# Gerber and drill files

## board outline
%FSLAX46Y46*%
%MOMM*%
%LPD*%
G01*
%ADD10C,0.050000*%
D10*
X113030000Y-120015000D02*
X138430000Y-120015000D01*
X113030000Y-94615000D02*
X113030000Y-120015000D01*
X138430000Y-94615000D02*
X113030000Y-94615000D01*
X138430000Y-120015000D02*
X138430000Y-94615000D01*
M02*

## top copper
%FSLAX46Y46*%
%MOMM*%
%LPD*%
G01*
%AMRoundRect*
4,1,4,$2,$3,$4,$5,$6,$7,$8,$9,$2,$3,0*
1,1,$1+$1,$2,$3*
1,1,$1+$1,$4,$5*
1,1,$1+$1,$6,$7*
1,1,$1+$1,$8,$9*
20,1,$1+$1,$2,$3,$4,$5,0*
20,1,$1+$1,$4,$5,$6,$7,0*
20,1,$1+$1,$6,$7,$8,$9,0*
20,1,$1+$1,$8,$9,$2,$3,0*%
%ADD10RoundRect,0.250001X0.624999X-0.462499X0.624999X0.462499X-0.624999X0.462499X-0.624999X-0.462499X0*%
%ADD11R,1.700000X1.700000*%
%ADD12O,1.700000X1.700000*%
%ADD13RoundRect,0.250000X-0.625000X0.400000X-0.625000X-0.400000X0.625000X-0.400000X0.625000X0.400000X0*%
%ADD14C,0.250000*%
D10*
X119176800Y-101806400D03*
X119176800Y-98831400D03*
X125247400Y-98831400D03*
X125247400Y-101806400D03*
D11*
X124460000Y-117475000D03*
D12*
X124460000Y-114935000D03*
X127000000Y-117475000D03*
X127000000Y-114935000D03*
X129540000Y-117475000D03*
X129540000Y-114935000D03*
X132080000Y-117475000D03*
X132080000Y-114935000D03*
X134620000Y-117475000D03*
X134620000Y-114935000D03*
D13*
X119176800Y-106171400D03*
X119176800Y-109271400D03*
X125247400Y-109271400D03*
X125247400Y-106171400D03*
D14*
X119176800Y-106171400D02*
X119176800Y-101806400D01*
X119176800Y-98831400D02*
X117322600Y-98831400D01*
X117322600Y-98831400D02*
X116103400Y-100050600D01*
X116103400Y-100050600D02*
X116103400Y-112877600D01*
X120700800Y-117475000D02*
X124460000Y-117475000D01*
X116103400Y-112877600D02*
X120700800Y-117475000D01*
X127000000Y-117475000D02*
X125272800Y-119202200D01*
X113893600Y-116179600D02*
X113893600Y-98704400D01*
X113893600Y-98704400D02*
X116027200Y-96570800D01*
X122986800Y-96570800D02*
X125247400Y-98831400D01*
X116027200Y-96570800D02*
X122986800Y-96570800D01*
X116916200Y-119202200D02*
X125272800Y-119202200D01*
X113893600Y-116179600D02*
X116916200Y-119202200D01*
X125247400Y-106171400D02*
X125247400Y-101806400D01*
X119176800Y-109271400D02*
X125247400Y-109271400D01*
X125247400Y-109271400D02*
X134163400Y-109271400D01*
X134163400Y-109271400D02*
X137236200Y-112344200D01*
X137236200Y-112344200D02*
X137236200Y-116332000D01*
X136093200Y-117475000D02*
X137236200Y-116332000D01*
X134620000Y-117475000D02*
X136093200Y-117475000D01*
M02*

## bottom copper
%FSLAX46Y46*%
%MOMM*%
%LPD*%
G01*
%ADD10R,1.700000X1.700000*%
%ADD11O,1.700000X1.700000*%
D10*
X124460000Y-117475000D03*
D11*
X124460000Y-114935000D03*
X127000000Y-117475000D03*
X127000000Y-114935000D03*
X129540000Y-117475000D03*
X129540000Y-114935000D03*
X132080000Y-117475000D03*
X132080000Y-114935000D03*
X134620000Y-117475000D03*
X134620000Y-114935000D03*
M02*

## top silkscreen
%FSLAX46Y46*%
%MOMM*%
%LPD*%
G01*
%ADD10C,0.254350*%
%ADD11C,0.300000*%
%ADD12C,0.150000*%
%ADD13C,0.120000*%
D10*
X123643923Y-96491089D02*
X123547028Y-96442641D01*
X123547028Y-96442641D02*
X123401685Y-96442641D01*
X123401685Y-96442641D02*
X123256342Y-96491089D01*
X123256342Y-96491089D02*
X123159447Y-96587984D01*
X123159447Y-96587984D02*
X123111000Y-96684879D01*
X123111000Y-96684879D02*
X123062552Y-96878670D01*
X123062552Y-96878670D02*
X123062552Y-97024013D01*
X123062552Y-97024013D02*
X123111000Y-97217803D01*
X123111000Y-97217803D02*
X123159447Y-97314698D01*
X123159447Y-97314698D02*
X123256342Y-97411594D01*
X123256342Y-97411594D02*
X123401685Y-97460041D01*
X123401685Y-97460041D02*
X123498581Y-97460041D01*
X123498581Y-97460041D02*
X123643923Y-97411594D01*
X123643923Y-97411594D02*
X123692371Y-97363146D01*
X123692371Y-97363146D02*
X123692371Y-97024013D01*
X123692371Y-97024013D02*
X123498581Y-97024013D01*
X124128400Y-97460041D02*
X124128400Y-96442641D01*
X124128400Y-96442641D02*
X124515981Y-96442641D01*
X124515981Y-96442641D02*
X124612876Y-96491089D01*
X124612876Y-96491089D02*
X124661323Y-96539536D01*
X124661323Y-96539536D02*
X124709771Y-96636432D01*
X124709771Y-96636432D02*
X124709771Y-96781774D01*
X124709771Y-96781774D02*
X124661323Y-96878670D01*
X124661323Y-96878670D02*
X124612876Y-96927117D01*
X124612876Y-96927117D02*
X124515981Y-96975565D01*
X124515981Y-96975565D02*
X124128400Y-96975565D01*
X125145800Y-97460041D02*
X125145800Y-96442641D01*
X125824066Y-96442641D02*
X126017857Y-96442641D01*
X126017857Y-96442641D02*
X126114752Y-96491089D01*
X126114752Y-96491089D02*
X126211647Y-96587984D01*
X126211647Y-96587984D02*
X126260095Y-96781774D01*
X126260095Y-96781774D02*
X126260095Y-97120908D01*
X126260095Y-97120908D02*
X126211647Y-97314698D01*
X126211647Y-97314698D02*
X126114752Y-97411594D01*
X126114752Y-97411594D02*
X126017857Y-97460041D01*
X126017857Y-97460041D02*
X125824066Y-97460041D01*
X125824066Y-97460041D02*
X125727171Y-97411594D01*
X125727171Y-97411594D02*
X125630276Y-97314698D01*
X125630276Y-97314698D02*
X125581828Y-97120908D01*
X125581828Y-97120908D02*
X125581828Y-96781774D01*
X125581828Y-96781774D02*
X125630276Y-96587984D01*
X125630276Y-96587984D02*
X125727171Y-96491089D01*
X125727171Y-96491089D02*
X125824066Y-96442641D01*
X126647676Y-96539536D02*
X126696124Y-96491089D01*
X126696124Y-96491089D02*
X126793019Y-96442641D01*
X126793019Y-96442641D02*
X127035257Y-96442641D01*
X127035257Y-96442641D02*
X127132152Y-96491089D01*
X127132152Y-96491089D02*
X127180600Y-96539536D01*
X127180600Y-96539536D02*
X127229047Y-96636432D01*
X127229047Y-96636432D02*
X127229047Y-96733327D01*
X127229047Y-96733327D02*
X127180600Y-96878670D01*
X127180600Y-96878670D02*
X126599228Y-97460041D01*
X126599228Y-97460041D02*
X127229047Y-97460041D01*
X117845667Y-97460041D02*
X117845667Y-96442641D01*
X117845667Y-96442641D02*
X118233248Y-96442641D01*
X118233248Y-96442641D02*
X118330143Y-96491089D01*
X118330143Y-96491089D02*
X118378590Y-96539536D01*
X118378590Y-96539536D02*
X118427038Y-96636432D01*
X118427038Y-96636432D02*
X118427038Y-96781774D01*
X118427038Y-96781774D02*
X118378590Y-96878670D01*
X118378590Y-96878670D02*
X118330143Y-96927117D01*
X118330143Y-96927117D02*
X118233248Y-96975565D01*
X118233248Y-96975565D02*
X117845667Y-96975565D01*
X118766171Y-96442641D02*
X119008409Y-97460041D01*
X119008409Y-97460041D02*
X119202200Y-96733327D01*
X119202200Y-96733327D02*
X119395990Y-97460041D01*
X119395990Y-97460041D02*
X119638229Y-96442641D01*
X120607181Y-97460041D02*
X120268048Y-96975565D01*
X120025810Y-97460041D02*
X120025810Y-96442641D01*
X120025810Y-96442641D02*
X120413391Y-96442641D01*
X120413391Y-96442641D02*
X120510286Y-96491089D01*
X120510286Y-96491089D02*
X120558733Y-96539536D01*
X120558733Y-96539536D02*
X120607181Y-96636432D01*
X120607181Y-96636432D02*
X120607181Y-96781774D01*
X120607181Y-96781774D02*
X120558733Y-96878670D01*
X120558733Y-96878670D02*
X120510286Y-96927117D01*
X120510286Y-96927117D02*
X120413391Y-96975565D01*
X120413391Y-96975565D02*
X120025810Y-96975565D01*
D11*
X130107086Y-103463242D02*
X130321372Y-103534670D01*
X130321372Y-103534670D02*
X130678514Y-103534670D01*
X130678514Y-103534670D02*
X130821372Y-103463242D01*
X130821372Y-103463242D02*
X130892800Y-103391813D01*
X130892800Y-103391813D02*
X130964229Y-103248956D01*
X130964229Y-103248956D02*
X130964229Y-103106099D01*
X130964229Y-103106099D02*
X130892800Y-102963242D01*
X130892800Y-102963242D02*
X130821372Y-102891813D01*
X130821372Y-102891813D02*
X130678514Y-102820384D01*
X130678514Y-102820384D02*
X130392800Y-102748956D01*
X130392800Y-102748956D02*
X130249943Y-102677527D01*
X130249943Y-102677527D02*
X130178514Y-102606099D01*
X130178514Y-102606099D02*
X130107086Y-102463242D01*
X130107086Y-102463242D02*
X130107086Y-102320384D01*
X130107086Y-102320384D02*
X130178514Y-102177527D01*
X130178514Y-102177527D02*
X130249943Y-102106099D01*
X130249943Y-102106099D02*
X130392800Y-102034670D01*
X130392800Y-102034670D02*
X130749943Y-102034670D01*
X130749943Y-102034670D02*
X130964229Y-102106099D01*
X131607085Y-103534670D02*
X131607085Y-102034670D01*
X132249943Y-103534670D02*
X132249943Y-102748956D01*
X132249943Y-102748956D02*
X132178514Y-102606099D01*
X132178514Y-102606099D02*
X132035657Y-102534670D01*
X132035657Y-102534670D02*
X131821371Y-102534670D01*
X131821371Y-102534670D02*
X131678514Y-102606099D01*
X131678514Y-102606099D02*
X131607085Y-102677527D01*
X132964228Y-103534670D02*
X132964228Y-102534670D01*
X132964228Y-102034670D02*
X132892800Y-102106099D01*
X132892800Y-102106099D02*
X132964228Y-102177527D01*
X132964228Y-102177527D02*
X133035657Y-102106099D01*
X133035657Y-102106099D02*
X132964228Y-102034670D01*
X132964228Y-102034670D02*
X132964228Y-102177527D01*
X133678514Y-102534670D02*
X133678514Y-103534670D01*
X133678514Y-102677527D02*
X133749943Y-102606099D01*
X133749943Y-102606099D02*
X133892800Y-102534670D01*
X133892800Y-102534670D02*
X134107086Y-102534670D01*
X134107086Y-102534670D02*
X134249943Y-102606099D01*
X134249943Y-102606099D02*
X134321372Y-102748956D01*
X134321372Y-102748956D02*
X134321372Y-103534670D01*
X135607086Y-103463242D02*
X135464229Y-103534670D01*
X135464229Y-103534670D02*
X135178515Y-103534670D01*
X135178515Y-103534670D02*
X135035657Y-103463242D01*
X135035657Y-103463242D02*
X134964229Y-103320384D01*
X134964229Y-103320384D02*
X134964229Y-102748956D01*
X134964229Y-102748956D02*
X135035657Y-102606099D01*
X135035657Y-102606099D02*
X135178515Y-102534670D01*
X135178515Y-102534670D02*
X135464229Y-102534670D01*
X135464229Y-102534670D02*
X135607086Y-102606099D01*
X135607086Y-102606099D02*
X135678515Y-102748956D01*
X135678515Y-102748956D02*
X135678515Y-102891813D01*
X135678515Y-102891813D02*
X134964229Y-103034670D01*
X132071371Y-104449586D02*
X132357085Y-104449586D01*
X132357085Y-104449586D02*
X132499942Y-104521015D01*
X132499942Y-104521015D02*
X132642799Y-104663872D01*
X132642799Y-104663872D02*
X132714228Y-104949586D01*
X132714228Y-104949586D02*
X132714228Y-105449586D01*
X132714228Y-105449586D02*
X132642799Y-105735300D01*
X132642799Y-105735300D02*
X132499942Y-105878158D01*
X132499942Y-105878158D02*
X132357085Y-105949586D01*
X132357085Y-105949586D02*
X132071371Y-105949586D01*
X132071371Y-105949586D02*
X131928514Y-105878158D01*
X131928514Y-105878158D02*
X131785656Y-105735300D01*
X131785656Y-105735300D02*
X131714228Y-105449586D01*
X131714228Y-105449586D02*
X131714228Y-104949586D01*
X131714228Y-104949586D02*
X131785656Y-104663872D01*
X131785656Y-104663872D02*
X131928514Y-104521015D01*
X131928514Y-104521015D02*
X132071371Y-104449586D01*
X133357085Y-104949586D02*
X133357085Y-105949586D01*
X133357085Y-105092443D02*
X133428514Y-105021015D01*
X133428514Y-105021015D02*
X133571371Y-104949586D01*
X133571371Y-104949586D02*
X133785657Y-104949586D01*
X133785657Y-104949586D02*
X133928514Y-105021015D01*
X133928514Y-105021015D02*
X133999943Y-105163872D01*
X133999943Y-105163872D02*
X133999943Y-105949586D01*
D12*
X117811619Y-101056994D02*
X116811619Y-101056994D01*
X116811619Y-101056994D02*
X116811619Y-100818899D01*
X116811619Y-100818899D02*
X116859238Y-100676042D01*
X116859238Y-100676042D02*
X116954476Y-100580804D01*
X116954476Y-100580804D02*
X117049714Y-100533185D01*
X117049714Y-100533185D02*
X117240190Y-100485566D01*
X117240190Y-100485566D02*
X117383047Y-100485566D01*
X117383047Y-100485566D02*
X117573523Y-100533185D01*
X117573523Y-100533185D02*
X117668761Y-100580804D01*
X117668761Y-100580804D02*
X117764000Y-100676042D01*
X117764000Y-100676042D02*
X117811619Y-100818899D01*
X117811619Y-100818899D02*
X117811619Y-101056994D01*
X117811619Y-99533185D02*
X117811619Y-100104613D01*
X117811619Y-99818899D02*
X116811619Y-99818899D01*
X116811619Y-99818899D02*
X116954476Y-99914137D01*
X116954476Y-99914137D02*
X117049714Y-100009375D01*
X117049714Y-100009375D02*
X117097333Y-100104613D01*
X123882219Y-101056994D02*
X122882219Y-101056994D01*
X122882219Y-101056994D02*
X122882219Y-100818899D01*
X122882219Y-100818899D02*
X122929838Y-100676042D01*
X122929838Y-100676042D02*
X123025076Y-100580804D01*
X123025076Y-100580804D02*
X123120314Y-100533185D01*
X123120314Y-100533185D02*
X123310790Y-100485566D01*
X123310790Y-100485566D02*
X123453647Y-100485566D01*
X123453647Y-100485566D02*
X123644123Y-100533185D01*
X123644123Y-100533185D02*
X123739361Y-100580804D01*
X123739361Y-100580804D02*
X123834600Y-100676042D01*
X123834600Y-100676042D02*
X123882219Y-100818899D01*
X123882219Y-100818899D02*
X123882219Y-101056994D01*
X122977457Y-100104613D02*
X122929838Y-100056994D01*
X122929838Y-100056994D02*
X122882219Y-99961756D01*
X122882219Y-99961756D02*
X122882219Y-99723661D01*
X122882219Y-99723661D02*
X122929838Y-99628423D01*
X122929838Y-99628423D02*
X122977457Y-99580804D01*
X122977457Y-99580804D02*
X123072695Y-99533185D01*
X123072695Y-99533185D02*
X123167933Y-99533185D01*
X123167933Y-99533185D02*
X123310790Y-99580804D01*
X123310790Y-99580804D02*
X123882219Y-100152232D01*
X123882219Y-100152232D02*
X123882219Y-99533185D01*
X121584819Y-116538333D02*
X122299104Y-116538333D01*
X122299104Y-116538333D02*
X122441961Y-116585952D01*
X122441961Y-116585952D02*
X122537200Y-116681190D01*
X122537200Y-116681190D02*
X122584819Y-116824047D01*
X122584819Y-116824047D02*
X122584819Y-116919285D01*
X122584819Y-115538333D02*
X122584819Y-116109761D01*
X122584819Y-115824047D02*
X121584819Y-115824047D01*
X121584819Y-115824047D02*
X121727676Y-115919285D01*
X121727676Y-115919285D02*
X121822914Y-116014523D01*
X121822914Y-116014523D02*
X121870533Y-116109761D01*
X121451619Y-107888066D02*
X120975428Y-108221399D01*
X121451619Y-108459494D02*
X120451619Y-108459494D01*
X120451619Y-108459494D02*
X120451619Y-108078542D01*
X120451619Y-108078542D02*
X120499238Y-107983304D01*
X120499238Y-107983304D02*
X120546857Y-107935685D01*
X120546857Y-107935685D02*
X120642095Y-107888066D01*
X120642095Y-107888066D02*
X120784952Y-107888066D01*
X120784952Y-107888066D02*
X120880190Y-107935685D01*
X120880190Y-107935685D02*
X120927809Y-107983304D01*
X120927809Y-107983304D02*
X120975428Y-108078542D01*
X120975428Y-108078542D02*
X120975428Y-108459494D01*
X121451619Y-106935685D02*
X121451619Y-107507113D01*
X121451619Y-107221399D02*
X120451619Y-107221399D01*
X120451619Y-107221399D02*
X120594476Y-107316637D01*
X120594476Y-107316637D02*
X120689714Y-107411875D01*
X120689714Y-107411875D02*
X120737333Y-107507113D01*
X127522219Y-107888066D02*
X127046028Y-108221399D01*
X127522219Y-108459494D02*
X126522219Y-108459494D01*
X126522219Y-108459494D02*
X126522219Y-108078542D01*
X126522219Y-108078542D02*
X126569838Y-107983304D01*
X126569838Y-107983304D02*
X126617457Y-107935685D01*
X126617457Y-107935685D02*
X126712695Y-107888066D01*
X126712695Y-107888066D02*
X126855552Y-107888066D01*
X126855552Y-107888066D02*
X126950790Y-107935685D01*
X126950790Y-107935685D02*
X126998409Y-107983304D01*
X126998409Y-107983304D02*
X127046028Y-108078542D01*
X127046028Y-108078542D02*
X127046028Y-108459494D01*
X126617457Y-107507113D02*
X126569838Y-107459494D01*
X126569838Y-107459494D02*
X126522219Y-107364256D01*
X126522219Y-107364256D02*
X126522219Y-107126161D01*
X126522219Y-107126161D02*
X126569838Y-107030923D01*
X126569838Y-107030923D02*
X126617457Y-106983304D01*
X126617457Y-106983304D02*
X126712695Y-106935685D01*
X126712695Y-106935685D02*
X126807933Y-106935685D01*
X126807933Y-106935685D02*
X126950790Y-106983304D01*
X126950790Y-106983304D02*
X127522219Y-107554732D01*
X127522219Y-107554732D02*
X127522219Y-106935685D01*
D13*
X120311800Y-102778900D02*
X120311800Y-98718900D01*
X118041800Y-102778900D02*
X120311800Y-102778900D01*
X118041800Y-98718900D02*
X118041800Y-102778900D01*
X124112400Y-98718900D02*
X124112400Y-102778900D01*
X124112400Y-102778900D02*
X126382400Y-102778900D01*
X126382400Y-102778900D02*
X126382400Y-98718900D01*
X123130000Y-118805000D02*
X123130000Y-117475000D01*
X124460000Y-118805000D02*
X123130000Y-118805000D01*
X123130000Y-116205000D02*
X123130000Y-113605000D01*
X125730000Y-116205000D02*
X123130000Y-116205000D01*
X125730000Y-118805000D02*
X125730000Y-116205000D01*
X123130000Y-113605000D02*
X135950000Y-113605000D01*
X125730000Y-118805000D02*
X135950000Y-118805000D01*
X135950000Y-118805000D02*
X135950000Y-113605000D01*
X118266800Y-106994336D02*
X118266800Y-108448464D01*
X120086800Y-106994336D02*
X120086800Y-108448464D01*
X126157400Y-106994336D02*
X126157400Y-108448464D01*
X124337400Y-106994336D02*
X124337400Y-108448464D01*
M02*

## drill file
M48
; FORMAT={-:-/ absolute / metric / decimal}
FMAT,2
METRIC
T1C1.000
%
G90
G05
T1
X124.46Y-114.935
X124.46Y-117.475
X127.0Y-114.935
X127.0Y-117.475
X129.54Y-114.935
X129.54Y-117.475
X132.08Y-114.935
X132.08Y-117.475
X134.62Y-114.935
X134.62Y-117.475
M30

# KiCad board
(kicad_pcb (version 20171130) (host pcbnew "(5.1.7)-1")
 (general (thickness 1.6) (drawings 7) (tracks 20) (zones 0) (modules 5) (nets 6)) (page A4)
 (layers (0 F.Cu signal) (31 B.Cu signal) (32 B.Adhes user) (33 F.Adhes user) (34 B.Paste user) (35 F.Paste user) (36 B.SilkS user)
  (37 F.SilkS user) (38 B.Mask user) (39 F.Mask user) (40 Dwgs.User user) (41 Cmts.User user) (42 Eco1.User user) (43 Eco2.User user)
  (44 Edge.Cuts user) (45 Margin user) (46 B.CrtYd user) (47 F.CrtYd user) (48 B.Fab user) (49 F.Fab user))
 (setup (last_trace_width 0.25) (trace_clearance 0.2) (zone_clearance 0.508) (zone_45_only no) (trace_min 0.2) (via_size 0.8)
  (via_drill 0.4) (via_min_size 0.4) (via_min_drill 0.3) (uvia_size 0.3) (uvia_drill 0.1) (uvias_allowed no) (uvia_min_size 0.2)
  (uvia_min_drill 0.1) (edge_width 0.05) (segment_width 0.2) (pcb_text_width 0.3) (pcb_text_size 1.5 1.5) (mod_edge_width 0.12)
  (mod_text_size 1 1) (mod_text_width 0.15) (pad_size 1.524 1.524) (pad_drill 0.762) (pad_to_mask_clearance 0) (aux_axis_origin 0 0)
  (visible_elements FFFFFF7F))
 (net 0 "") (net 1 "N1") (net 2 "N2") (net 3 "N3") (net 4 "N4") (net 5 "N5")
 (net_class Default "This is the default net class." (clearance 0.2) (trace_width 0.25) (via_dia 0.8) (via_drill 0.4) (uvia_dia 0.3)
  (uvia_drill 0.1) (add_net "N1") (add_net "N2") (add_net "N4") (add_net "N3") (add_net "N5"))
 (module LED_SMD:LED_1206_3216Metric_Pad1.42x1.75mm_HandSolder (layer F.Cu) (at 119.1768 100.3189 90)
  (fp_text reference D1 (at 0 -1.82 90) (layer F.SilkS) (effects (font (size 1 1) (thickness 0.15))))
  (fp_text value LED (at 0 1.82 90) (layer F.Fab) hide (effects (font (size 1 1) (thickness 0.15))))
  (fp_line (start -2.46 1.135) (end 1.6 1.135) (layer F.SilkS) (width 0.12))
  (fp_line (start -2.46 -1.135) (end -2.46 1.135) (layer F.SilkS) (width 0.12))
  (fp_line (start 1.6 -1.135) (end -2.46 -1.135) (layer F.SilkS) (width 0.12))
  (pad 1 smd roundrect (at -1.4875 0 90) (size 1.425 1.75) (layers F.Cu F.Paste F.Mask) (roundrect_rratio 0.175439) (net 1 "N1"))
  (pad 2 smd roundrect (at 1.4875 0 90) (size 1.425 1.75) (layers F.Cu F.Paste F.Mask) (roundrect_rratio 0.175439) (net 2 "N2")))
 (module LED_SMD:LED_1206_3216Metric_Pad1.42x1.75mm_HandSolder (layer F.Cu) (at 125.2474 100.3189 90)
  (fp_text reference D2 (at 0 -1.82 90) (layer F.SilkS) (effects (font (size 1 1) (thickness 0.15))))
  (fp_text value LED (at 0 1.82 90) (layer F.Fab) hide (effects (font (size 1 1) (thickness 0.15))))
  (fp_line (start 1.6 -1.135) (end -2.46 -1.135) (layer F.SilkS) (width 0.12))
  (fp_line (start -2.46 -1.135) (end -2.46 1.135) (layer F.SilkS) (width 0.12))
  (fp_line (start -2.46 1.135) (end 1.6 1.135) (layer F.SilkS) (width 0.12))
  (pad 2 smd roundrect (at 1.4875 0 90) (size 1.425 1.75) (layers F.Cu F.Paste F.Mask) (roundrect_rratio 0.175439) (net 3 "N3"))
  (pad 1 smd roundrect (at -1.4875 0 90) (size 1.425 1.75) (layers F.Cu F.Paste F.Mask) (roundrect_rratio 0.175439) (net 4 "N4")))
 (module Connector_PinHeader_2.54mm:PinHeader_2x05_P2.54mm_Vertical (layer F.Cu) (at 124.46 117.475 90)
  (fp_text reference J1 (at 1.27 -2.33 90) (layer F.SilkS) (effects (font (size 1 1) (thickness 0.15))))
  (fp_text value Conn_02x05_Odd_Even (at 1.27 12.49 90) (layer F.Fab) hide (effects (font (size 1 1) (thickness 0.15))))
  (fp_line (start -1.33 -1.33) (end 0 -1.33) (layer F.SilkS) (width 0.12))
  (fp_line (start -1.33 0) (end -1.33 -1.33) (layer F.SilkS) (width 0.12))
  (fp_line (start 1.27 -1.33) (end 3.87 -1.33) (layer F.SilkS) (width 0.12))
  (fp_line (start 1.27 1.27) (end 1.27 -1.33) (layer F.SilkS) (width 0.12))
  (fp_line (start -1.33 1.27) (end 1.27 1.27) (layer F.SilkS) (width 0.12))
  (fp_line (start 3.87 -1.33) (end 3.87 11.49) (layer F.SilkS) (width 0.12))
  (fp_line (start -1.33 1.27) (end -1.33 11.49) (layer F.SilkS) (width 0.12))
  (fp_line (start -1.33 11.49) (end 3.87 11.49) (layer F.SilkS) (width 0.12))
  (pad 1 thru_hole rect (at 0 0 90) (size 1.7 1.7) (drill 1) (layers *.Cu *.Mask) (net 2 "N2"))
  (pad 2 thru_hole oval (at 2.54 0 90) (size 1.7 1.7) (drill 1) (layers *.Cu *.Mask))
  (pad 3 thru_hole oval (at 0 2.54 90) (size 1.7 1.7) (drill 1) (layers *.Cu *.Mask) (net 3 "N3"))
  (pad 4 thru_hole oval (at 2.54 2.54 90) (size 1.7 1.7) (drill 1) (layers *.Cu *.Mask))
  (pad 5 thru_hole oval (at 0 5.08 90) (size 1.7 1.7) (drill 1) (layers *.Cu *.Mask))
  (pad 6 thru_hole oval (at 2.54 5.08 90) (size 1.7 1.7) (drill 1) (layers *.Cu *.Mask))
  (pad 7 thru_hole oval (at 0 7.62 90) (size 1.7 1.7) (drill 1) (layers *.Cu *.Mask))
  (pad 8 thru_hole oval (at 2.54 7.62 90) (size 1.7 1.7) (drill 1) (layers *.Cu *.Mask))
  (pad 9 thru_hole oval (at 0 10.16 90) (size 1.7 1.7) (drill 1) (layers *.Cu *.Mask) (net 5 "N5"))
  (pad 10 thru_hole oval (at 2.54 10.16 90) (size 1.7 1.7) (drill 1) (layers *.Cu *.Mask)))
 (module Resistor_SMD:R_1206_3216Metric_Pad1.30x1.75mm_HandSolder (layer F.Cu) (at 119.1768 107.7214 270)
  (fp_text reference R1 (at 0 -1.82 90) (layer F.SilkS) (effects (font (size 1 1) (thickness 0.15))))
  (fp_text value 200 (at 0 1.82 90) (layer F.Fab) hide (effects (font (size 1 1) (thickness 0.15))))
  (fp_line (start -0.727064 0.91) (end 0.727064 0.91) (layer F.SilkS) (width 0.12))
  (fp_line (start -0.727064 -0.91) (end 0.727064 -0.91) (layer F.SilkS) (width 0.12))
  (pad 1 smd roundrect (at -1.55 0 270) (size 1.3 1.75) (layers F.Cu F.Paste F.Mask) (roundrect_rratio 0.192308) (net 1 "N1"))
  (pad 2 smd roundrect (at 1.55 0 270) (size 1.3 1.75) (layers F.Cu F.Paste F.Mask) (roundrect_rratio 0.192308) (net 5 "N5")))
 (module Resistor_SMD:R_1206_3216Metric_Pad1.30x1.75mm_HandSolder (layer F.Cu) (at 125.2474 107.7214 270)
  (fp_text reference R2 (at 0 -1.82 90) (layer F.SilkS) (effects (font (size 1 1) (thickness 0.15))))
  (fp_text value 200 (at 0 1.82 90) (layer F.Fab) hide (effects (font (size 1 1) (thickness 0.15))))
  (fp_line (start -0.727064 -0.91) (end 0.727064 -0.91) (layer F.SilkS) (width 0.12))
  (fp_line (start -0.727064 0.91) (end 0.727064 0.91) (layer F.SilkS) (width 0.12))
  (pad 2 smd roundrect (at 1.55 0 270) (size 1.3 1.75) (layers F.Cu F.Paste F.Mask) (roundrect_rratio 0.192308) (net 5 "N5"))
  (pad 1 smd roundrect (at -1.55 0 270) (size 1.3 1.75) (layers F.Cu F.Paste F.Mask) (roundrect_rratio 0.192308) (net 4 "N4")))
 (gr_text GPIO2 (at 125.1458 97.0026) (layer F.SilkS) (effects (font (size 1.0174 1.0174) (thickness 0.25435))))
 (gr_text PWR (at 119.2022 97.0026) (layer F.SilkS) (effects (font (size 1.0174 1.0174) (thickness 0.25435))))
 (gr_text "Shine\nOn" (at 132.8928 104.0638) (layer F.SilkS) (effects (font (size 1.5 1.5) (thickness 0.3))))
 (gr_line (start 113.03 120.015) (end 138.43 120.015) (layer Edge.Cuts) (width 0.05))
 (gr_line (start 113.03 94.615) (end 113.03 120.015) (layer Edge.Cuts) (width 0.05))
 (gr_line (start 138.43 94.615) (end 113.03 94.615) (layer Edge.Cuts) (width 0.05))
 (gr_line (start 138.43 120.015) (end 138.43 94.615) (layer Edge.Cuts) (width 0.05))
 (segment (start 119.1768 106.1714) (end 119.1768 101.8064) (width 0.25) (layer F.Cu) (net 1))
 (segment (start 119.1768 98.8314) (end 117.3226 98.8314) (width 0.25) (layer F.Cu) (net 2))
 (segment (start 117.3226 98.8314) (end 116.1034 100.0506) (width 0.25) (layer F.Cu) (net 2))
 (segment (start 116.1034 100.0506) (end 116.1034 112.8776) (width 0.25) (layer F.Cu) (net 2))
 (segment (start 120.7008 117.475) (end 124.46 117.475) (width 0.25) (layer F.Cu) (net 2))
 (segment (start 116.1034 112.8776) (end 120.7008 117.475) (width 0.25) (layer F.Cu) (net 2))
 (segment (start 127 117.475) (end 125.2728 119.2022) (width 0.25) (layer F.Cu) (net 3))
 (segment (start 113.8936 116.1796) (end 113.8936 98.7044) (width 0.25) (layer F.Cu) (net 3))
 (segment (start 113.8936 98.7044) (end 116.0272 96.5708) (width 0.25) (layer F.Cu) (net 3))
 (segment (start 122.9868 96.5708) (end 125.2474 98.8314) (width 0.25) (layer F.Cu) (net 3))
 (segment (start 116.0272 96.5708) (end 122.9868 96.5708) (width 0.25) (layer F.Cu) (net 3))
 (segment (start 116.9162 119.2022) (end 125.2728 119.2022) (width 0.25) (layer F.Cu) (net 3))
 (segment (start 113.8936 116.1796) (end 116.9162 119.2022) (width 0.25) (layer F.Cu) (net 3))
 (segment (start 125.2474 106.1714) (end 125.2474 101.8064) (width 0.25) (layer F.Cu) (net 4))
 (segment (start 119.1768 109.2714) (end 125.2474 109.2714) (width 0.25) (layer F.Cu) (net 5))
 (segment (start 125.2474 109.2714) (end 134.1634 109.2714) (width 0.25) (layer F.Cu) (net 5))
 (segment (start 134.1634 109.2714) (end 137.2362 112.3442) (width 0.25) (layer F.Cu) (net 5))
 (segment (start 137.2362 112.3442) (end 137.2362 116.332) (width 0.25) (layer F.Cu) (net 5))
 (segment (start 136.0932 117.475) (end 137.2362 116.332) (width 0.25) (layer F.Cu) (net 5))
 (segment (start 134.62 117.475) (end 136.0932 117.475) (width 0.25) (layer F.Cu) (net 5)))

